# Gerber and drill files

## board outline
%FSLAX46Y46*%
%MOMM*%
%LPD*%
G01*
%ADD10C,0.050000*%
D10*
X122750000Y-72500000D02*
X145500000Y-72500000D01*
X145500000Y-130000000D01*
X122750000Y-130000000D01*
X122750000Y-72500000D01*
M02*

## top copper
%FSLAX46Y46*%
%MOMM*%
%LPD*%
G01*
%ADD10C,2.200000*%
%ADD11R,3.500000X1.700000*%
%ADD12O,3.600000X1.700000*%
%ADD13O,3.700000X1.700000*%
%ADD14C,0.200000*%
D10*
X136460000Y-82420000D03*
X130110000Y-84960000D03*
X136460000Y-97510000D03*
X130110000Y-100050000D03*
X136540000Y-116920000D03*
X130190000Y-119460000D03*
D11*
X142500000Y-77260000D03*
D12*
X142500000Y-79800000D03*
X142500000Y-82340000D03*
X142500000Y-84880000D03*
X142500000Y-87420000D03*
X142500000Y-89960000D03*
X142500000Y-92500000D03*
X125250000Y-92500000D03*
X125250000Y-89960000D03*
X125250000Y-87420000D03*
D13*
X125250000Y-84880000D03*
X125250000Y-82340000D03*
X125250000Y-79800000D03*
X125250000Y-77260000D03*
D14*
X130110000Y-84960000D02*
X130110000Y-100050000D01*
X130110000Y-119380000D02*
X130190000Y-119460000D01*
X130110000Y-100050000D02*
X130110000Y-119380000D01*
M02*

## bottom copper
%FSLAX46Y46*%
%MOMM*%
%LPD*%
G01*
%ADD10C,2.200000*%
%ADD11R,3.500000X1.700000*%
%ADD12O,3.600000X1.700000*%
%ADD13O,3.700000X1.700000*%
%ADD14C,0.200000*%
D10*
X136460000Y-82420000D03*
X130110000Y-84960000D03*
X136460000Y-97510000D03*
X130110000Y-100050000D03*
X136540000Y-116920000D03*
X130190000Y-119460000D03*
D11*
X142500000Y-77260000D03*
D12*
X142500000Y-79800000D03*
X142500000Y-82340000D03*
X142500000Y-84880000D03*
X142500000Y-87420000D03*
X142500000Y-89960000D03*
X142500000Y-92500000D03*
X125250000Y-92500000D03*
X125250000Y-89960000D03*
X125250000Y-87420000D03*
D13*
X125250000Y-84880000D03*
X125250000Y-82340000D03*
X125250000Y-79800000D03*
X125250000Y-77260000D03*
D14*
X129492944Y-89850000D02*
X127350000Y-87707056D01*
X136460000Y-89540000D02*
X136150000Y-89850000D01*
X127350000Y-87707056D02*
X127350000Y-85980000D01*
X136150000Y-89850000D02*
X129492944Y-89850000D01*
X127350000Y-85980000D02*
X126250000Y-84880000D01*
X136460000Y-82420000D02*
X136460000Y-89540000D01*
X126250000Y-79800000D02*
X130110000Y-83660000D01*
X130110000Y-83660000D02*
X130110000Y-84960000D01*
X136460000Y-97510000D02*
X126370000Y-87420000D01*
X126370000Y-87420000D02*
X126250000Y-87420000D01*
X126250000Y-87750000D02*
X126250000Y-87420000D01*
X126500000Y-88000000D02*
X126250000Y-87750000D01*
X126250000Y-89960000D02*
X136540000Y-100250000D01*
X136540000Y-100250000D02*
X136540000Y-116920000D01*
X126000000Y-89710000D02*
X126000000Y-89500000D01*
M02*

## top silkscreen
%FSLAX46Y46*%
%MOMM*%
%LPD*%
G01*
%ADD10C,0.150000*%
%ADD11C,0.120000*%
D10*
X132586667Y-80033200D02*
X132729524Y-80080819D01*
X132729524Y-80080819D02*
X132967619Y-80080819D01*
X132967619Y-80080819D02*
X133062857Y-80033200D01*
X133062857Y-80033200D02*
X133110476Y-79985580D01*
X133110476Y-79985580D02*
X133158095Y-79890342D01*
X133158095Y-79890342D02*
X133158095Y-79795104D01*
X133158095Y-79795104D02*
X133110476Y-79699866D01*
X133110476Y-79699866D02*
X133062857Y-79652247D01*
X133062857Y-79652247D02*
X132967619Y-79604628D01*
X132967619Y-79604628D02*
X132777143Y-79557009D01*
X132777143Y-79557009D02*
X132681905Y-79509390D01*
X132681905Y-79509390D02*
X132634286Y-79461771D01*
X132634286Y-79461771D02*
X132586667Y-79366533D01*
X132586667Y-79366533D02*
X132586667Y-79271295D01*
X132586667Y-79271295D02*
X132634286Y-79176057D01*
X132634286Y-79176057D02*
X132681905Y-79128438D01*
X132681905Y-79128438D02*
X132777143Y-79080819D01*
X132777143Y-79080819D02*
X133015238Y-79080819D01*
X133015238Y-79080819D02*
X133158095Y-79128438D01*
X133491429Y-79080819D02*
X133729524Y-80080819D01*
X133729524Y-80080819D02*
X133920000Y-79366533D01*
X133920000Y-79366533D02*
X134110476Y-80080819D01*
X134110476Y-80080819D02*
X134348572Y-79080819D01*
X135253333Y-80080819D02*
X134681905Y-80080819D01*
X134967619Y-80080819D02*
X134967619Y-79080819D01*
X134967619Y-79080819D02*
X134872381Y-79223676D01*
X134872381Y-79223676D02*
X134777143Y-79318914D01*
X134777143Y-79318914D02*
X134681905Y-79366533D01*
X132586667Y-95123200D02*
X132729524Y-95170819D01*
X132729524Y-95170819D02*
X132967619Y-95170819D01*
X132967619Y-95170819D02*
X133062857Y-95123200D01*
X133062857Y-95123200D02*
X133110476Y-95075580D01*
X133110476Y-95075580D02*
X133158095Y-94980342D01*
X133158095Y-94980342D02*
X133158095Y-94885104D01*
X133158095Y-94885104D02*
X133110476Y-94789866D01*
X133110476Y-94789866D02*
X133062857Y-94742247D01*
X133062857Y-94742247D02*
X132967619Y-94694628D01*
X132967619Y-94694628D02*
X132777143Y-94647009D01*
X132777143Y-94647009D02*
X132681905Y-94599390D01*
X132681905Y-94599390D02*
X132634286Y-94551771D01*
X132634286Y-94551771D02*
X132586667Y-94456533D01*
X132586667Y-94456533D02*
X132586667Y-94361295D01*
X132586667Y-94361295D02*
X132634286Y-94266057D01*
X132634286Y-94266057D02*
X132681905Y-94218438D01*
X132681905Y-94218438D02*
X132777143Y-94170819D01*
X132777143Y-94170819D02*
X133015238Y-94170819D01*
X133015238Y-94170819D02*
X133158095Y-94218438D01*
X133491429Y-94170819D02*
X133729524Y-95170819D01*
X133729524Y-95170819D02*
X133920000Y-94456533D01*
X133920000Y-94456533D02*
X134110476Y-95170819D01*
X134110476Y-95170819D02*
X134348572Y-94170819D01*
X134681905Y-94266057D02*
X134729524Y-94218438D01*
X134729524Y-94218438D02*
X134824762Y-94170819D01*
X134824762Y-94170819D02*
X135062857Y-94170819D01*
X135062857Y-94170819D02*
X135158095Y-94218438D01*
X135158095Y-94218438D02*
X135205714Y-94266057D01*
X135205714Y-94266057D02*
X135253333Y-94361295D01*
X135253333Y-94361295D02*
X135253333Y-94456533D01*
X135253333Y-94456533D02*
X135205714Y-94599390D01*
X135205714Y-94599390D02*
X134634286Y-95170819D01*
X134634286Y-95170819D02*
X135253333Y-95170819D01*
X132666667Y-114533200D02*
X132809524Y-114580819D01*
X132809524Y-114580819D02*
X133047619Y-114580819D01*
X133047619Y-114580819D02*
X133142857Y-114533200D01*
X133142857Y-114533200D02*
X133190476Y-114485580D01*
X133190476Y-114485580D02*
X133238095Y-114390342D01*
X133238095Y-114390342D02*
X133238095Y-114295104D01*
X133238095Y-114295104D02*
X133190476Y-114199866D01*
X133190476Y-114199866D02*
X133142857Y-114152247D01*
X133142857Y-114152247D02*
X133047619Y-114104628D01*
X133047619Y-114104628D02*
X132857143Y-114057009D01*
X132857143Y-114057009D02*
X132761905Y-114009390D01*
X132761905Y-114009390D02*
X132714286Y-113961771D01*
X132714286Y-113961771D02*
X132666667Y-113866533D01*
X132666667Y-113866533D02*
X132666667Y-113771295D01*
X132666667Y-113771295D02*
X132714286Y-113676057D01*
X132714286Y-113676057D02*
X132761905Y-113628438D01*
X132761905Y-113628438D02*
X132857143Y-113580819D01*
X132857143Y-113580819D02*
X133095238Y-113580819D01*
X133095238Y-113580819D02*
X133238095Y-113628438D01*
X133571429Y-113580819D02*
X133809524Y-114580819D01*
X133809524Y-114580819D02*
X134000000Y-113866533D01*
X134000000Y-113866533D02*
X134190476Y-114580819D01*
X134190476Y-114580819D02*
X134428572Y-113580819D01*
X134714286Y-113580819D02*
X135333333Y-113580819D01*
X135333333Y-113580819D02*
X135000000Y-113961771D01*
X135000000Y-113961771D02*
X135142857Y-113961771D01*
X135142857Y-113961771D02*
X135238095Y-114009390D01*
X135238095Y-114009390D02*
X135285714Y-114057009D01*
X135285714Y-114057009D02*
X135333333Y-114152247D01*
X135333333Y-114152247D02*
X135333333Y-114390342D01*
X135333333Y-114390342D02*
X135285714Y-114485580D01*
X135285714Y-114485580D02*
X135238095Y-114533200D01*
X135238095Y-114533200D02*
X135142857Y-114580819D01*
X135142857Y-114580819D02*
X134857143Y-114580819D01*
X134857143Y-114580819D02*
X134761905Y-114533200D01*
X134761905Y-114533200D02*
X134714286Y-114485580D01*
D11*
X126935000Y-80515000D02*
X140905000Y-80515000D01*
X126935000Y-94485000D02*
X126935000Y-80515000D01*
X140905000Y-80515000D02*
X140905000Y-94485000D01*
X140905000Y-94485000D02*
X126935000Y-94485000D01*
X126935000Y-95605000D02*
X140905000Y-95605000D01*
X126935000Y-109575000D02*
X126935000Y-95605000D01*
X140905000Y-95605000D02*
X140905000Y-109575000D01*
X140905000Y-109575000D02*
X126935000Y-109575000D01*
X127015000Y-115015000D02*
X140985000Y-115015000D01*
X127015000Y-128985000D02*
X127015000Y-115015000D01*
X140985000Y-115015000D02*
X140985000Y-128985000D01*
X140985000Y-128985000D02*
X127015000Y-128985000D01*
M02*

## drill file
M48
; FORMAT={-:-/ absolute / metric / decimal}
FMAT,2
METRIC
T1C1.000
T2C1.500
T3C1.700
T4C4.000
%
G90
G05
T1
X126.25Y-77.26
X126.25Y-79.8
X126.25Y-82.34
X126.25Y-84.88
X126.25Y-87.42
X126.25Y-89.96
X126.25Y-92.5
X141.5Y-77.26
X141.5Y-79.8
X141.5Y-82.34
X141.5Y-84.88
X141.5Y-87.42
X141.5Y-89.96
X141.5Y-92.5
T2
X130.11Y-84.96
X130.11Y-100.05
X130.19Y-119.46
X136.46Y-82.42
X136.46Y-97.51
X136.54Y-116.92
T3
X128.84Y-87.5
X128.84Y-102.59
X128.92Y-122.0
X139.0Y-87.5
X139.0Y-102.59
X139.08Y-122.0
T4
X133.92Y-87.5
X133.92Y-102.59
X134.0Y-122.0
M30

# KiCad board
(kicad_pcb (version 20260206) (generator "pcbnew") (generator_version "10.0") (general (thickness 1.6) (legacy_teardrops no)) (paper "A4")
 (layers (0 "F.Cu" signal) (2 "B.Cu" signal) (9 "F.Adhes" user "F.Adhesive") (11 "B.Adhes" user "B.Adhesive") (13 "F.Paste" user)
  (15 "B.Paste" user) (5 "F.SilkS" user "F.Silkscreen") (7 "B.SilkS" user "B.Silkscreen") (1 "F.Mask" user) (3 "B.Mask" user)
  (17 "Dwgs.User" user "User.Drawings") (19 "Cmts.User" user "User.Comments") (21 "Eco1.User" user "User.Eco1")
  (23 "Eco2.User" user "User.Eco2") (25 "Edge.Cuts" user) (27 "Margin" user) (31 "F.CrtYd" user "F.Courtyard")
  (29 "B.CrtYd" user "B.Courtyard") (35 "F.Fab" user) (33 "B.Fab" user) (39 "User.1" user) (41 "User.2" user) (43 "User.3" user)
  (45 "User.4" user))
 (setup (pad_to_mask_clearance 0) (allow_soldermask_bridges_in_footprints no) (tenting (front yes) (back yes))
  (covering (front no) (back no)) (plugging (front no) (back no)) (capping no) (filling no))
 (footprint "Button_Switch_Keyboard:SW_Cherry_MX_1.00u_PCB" (layer "F.Cu") (at 136.46 82.42)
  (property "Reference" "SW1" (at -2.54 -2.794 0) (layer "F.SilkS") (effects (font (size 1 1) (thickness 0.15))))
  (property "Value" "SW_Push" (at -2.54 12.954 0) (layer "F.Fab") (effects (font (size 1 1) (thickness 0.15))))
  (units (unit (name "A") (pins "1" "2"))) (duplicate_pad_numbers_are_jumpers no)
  (fp_line (start -9.525 -1.905) (end 4.445 -1.905) (stroke (width 0.12) (type solid)) (layer "F.SilkS"))
  (fp_line (start -9.525 12.065) (end -9.525 -1.905) (stroke (width 0.12) (type solid)) (layer "F.SilkS"))
  (fp_line (start 4.445 -1.905) (end 4.445 12.065) (stroke (width 0.12) (type solid)) (layer "F.SilkS"))
  (fp_line (start 4.445 12.065) (end -9.525 12.065) (stroke (width 0.12) (type solid)) (layer "F.SilkS"))
  (pad "" np_thru_hole circle (at -7.62 5.08) (size 1.7 1.7) (drill 1.7) (layers "*.Cu" "*.Mask"))
  (pad "" np_thru_hole circle (at -2.54 5.08) (size 4 4) (drill 4) (layers "*.Cu" "*.Mask"))
  (pad "" np_thru_hole circle (at 2.54 5.08) (size 1.7 1.7) (drill 1.7) (layers "*.Cu" "*.Mask"))
  (pad "1" thru_hole circle (at 0 0) (size 2.2 2.2) (drill 1.5) (layers "*.Cu" "*.Mask") (remove_unused_layers no)
   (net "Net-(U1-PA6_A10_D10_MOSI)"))
  (pad "2" thru_hole circle (at -6.35 2.54) (size 2.2 2.2) (drill 1.5) (layers "*.Cu" "*.Mask") (remove_unused_layers no) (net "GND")))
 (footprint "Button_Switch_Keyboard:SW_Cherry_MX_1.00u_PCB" (layer "F.Cu") (at 136.46 97.51)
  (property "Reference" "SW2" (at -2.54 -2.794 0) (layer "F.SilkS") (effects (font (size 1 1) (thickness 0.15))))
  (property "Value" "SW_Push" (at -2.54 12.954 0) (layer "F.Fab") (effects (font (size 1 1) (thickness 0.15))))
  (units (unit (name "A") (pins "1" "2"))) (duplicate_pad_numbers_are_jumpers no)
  (fp_line (start -9.525 -1.905) (end 4.445 -1.905) (stroke (width 0.12) (type solid)) (layer "F.SilkS"))
  (fp_line (start -9.525 12.065) (end -9.525 -1.905) (stroke (width 0.12) (type solid)) (layer "F.SilkS"))
  (fp_line (start 4.445 -1.905) (end 4.445 12.065) (stroke (width 0.12) (type solid)) (layer "F.SilkS"))
  (fp_line (start 4.445 12.065) (end -9.525 12.065) (stroke (width 0.12) (type solid)) (layer "F.SilkS"))
  (pad "" np_thru_hole circle (at -7.62 5.08) (size 1.7 1.7) (drill 1.7) (layers "*.Cu" "*.Mask"))
  (pad "" np_thru_hole circle (at -2.54 5.08) (size 4 4) (drill 4) (layers "*.Cu" "*.Mask"))
  (pad "" np_thru_hole circle (at 2.54 5.08) (size 1.7 1.7) (drill 1.7) (layers "*.Cu" "*.Mask"))
  (pad "1" thru_hole circle (at 0 0) (size 2.2 2.2) (drill 1.5) (layers "*.Cu" "*.Mask") (remove_unused_layers no)
   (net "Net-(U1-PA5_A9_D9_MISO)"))
  (pad "2" thru_hole circle (at -6.35 2.54) (size 2.2 2.2) (drill 1.5) (layers "*.Cu" "*.Mask") (remove_unused_layers no) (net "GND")))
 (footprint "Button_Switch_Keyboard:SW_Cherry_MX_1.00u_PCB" (layer "F.Cu") (at 136.54 116.92)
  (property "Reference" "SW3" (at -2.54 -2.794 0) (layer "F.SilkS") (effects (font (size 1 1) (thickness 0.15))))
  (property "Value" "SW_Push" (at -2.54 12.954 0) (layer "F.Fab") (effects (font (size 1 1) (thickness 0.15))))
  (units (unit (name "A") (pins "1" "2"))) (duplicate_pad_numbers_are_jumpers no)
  (fp_line (start -9.525 -1.905) (end 4.445 -1.905) (stroke (width 0.12) (type solid)) (layer "F.SilkS"))
  (fp_line (start -9.525 12.065) (end -9.525 -1.905) (stroke (width 0.12) (type solid)) (layer "F.SilkS"))
  (fp_line (start 4.445 -1.905) (end 4.445 12.065) (stroke (width 0.12) (type solid)) (layer "F.SilkS"))
  (fp_line (start 4.445 12.065) (end -9.525 12.065) (stroke (width 0.12) (type solid)) (layer "F.SilkS"))
  (pad "" np_thru_hole circle (at -7.62 5.08) (size 1.7 1.7) (drill 1.7) (layers "*.Cu" "*.Mask"))
  (pad "" np_thru_hole circle (at -2.54 5.08) (size 4 4) (drill 4) (layers "*.Cu" "*.Mask"))
  (pad "" np_thru_hole circle (at 2.54 5.08) (size 1.7 1.7) (drill 1.7) (layers "*.Cu" "*.Mask"))
  (pad "1" thru_hole circle (at 0 0) (size 2.2 2.2) (drill 1.5) (layers "*.Cu" "*.Mask") (remove_unused_layers no)
   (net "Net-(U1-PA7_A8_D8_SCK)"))
  (pad "2" thru_hole circle (at -6.35 2.54) (size 2.2 2.2) (drill 1.5) (layers "*.Cu" "*.Mask") (remove_unused_layers no) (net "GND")))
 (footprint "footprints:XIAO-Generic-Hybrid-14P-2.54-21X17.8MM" (layer "B.Cu") (at 133.875 84.88 180)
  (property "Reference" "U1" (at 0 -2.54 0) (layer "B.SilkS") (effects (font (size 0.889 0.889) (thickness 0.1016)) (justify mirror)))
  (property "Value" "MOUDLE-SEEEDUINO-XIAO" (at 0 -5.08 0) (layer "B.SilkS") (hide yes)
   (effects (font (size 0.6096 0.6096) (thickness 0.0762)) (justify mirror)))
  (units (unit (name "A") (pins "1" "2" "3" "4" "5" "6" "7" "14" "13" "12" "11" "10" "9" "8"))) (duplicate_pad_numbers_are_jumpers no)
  (pad "1" thru_hole rect (at -7.625 7.62 180) (size 3.5 1.7) (drill 1 (offset -1 0)) (layers "*.Cu" "*.Mask") (remove_unused_layers no)
   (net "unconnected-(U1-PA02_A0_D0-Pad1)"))
  (pad "2" thru_hole oval (at -7.625 5.08 180) (size 3.6 1.7) (drill 1 (offset -1 0)) (layers "*.Cu" "*.Mask") (remove_unused_layers no)
   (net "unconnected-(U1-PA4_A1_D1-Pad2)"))
  (pad "3" thru_hole oval (at -7.625 2.54 180) (size 3.6 1.7) (drill 1 (offset -1 0)) (layers "*.Cu" "*.Mask") (remove_unused_layers no)
   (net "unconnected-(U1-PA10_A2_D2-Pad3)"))
  (pad "4" thru_hole oval (at -7.625 0 180) (size 3.6 1.7) (drill 1 (offset -1 0)) (layers "*.Cu" "*.Mask") (remove_unused_layers no)
   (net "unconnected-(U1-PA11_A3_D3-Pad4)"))
  (pad "5" thru_hole oval (at -7.625 -2.54 180) (size 3.6 1.7) (drill 1 (offset -1 0)) (layers "*.Cu" "*.Mask") (remove_unused_layers no)
   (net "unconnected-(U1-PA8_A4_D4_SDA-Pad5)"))
  (pad "6" thru_hole oval (at -7.625 -5.08) (size 3.6 1.7) (drill 1 (offset 1 0)) (layers "*.Cu" "*.Mask") (remove_unused_layers no)
   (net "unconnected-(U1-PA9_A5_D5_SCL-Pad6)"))
  (pad "7" thru_hole oval (at -7.625 -7.62 180) (size 3.6 1.7) (drill 1 (offset -1 0)) (layers "*.Cu" "*.Mask") (remove_unused_layers no)
   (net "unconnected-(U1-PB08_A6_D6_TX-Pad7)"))
  (pad "8" thru_hole oval (at 7.625 -7.62 180) (size 3.6 1.7) (drill 1 (offset 1 0)) (layers "*.Cu" "*.Mask") (remove_unused_layers no)
   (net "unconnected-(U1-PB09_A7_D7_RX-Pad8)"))
  (pad "9" thru_hole oval (at 7.625 -5.08 180) (size 3.6 1.7) (drill 1 (offset 1 0)) (layers "*.Cu" "*.Mask") (remove_unused_layers no)
   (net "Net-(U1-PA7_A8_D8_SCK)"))
  (pad "10" thru_hole oval (at 7.625 -2.54 180) (size 3.6 1.7) (drill 1 (offset 1 0)) (layers "*.Cu" "*.Mask") (remove_unused_layers no)
   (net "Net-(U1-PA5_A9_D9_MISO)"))
  (pad "11" thru_hole oval (at 7.625 0 180) (size 3.7 1.7) (drill 1 (offset 1 0)) (layers "*.Cu" "*.Mask") (remove_unused_layers no)
   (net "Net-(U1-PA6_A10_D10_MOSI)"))
  (pad "12" thru_hole oval (at 7.625 2.54 180) (size 3.7 1.7) (drill 1 (offset 1 0)) (layers "*.Cu" "*.Mask") (remove_unused_layers no)
   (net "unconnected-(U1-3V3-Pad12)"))
  (pad "13" thru_hole oval (at 7.625 5.08 180) (size 3.7 1.7) (drill 1 (offset 1 0)) (layers "*.Cu" "*.Mask") (remove_unused_layers no)
   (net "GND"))
  (pad "14" thru_hole oval (at 7.625 7.62 180) (size 3.7 1.7) (drill 1 (offset 1 0)) (layers "*.Cu" "*.Mask") (remove_unused_layers no)
   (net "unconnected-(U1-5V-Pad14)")))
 (gr_rect (start 122.75 72.5) (end 145.5 130) (stroke (width 0.05) (type default)) (fill no) (layer "Edge.Cuts"))
 (segment (start 129.492944 89.85) (end 127.35 87.707056) (width 0.2) (layer "B.Cu") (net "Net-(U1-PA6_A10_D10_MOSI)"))
 (segment (start 136.46 89.54) (end 136.15 89.85) (width 0.2) (layer "B.Cu") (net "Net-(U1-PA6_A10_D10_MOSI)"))
 (segment (start 127.35 87.707056) (end 127.35 85.98) (width 0.2) (layer "B.Cu") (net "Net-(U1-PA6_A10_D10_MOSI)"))
 (segment (start 136.15 89.85) (end 129.492944 89.85) (width 0.2) (layer "B.Cu") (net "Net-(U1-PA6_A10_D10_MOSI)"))
 (segment (start 127.35 85.98) (end 126.25 84.88) (width 0.2) (layer "B.Cu") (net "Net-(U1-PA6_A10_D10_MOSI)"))
 (segment (start 136.46 82.42) (end 136.46 89.54) (width 0.2) (layer "B.Cu") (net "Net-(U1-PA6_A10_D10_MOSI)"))
 (segment (start 130.11 84.96) (end 130.11 100.05) (width 0.2) (layer "F.Cu") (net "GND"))
 (segment (start 130.11 119.38) (end 130.19 119.46) (width 0.2) (layer "F.Cu") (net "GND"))
 (segment (start 130.11 100.05) (end 130.11 119.38) (width 0.2) (layer "F.Cu") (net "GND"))
 (segment (start 126.25 79.8) (end 130.11 83.66) (width 0.2) (layer "B.Cu") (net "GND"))
 (segment (start 130.11 83.66) (end 130.11 84.96) (width 0.2) (layer "B.Cu") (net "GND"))
 (segment (start 136.46 97.51) (end 126.37 87.42) (width 0.2) (layer "B.Cu") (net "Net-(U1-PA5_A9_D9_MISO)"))
 (segment (start 126.37 87.42) (end 126.25 87.42) (width 0.2) (layer "B.Cu") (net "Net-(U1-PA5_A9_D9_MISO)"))
 (segment (start 126.25 87.75) (end 126.25 87.42) (width 0.2) (layer "B.Cu") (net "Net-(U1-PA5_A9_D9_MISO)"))
 (segment (start 126.5 88) (end 126.25 87.75) (width 0.2) (layer "B.Cu") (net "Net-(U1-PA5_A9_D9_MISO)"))
 (segment (start 126.25 89.96) (end 136.54 100.25) (width 0.2) (layer "B.Cu") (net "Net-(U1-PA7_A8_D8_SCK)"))
 (segment (start 136.54 100.25) (end 136.54 116.92) (width 0.2) (layer "B.Cu") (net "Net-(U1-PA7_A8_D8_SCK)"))
 (segment (start 126 89.71) (end 126 89.5) (width 0.2) (layer "B.Cu") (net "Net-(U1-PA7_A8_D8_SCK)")))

